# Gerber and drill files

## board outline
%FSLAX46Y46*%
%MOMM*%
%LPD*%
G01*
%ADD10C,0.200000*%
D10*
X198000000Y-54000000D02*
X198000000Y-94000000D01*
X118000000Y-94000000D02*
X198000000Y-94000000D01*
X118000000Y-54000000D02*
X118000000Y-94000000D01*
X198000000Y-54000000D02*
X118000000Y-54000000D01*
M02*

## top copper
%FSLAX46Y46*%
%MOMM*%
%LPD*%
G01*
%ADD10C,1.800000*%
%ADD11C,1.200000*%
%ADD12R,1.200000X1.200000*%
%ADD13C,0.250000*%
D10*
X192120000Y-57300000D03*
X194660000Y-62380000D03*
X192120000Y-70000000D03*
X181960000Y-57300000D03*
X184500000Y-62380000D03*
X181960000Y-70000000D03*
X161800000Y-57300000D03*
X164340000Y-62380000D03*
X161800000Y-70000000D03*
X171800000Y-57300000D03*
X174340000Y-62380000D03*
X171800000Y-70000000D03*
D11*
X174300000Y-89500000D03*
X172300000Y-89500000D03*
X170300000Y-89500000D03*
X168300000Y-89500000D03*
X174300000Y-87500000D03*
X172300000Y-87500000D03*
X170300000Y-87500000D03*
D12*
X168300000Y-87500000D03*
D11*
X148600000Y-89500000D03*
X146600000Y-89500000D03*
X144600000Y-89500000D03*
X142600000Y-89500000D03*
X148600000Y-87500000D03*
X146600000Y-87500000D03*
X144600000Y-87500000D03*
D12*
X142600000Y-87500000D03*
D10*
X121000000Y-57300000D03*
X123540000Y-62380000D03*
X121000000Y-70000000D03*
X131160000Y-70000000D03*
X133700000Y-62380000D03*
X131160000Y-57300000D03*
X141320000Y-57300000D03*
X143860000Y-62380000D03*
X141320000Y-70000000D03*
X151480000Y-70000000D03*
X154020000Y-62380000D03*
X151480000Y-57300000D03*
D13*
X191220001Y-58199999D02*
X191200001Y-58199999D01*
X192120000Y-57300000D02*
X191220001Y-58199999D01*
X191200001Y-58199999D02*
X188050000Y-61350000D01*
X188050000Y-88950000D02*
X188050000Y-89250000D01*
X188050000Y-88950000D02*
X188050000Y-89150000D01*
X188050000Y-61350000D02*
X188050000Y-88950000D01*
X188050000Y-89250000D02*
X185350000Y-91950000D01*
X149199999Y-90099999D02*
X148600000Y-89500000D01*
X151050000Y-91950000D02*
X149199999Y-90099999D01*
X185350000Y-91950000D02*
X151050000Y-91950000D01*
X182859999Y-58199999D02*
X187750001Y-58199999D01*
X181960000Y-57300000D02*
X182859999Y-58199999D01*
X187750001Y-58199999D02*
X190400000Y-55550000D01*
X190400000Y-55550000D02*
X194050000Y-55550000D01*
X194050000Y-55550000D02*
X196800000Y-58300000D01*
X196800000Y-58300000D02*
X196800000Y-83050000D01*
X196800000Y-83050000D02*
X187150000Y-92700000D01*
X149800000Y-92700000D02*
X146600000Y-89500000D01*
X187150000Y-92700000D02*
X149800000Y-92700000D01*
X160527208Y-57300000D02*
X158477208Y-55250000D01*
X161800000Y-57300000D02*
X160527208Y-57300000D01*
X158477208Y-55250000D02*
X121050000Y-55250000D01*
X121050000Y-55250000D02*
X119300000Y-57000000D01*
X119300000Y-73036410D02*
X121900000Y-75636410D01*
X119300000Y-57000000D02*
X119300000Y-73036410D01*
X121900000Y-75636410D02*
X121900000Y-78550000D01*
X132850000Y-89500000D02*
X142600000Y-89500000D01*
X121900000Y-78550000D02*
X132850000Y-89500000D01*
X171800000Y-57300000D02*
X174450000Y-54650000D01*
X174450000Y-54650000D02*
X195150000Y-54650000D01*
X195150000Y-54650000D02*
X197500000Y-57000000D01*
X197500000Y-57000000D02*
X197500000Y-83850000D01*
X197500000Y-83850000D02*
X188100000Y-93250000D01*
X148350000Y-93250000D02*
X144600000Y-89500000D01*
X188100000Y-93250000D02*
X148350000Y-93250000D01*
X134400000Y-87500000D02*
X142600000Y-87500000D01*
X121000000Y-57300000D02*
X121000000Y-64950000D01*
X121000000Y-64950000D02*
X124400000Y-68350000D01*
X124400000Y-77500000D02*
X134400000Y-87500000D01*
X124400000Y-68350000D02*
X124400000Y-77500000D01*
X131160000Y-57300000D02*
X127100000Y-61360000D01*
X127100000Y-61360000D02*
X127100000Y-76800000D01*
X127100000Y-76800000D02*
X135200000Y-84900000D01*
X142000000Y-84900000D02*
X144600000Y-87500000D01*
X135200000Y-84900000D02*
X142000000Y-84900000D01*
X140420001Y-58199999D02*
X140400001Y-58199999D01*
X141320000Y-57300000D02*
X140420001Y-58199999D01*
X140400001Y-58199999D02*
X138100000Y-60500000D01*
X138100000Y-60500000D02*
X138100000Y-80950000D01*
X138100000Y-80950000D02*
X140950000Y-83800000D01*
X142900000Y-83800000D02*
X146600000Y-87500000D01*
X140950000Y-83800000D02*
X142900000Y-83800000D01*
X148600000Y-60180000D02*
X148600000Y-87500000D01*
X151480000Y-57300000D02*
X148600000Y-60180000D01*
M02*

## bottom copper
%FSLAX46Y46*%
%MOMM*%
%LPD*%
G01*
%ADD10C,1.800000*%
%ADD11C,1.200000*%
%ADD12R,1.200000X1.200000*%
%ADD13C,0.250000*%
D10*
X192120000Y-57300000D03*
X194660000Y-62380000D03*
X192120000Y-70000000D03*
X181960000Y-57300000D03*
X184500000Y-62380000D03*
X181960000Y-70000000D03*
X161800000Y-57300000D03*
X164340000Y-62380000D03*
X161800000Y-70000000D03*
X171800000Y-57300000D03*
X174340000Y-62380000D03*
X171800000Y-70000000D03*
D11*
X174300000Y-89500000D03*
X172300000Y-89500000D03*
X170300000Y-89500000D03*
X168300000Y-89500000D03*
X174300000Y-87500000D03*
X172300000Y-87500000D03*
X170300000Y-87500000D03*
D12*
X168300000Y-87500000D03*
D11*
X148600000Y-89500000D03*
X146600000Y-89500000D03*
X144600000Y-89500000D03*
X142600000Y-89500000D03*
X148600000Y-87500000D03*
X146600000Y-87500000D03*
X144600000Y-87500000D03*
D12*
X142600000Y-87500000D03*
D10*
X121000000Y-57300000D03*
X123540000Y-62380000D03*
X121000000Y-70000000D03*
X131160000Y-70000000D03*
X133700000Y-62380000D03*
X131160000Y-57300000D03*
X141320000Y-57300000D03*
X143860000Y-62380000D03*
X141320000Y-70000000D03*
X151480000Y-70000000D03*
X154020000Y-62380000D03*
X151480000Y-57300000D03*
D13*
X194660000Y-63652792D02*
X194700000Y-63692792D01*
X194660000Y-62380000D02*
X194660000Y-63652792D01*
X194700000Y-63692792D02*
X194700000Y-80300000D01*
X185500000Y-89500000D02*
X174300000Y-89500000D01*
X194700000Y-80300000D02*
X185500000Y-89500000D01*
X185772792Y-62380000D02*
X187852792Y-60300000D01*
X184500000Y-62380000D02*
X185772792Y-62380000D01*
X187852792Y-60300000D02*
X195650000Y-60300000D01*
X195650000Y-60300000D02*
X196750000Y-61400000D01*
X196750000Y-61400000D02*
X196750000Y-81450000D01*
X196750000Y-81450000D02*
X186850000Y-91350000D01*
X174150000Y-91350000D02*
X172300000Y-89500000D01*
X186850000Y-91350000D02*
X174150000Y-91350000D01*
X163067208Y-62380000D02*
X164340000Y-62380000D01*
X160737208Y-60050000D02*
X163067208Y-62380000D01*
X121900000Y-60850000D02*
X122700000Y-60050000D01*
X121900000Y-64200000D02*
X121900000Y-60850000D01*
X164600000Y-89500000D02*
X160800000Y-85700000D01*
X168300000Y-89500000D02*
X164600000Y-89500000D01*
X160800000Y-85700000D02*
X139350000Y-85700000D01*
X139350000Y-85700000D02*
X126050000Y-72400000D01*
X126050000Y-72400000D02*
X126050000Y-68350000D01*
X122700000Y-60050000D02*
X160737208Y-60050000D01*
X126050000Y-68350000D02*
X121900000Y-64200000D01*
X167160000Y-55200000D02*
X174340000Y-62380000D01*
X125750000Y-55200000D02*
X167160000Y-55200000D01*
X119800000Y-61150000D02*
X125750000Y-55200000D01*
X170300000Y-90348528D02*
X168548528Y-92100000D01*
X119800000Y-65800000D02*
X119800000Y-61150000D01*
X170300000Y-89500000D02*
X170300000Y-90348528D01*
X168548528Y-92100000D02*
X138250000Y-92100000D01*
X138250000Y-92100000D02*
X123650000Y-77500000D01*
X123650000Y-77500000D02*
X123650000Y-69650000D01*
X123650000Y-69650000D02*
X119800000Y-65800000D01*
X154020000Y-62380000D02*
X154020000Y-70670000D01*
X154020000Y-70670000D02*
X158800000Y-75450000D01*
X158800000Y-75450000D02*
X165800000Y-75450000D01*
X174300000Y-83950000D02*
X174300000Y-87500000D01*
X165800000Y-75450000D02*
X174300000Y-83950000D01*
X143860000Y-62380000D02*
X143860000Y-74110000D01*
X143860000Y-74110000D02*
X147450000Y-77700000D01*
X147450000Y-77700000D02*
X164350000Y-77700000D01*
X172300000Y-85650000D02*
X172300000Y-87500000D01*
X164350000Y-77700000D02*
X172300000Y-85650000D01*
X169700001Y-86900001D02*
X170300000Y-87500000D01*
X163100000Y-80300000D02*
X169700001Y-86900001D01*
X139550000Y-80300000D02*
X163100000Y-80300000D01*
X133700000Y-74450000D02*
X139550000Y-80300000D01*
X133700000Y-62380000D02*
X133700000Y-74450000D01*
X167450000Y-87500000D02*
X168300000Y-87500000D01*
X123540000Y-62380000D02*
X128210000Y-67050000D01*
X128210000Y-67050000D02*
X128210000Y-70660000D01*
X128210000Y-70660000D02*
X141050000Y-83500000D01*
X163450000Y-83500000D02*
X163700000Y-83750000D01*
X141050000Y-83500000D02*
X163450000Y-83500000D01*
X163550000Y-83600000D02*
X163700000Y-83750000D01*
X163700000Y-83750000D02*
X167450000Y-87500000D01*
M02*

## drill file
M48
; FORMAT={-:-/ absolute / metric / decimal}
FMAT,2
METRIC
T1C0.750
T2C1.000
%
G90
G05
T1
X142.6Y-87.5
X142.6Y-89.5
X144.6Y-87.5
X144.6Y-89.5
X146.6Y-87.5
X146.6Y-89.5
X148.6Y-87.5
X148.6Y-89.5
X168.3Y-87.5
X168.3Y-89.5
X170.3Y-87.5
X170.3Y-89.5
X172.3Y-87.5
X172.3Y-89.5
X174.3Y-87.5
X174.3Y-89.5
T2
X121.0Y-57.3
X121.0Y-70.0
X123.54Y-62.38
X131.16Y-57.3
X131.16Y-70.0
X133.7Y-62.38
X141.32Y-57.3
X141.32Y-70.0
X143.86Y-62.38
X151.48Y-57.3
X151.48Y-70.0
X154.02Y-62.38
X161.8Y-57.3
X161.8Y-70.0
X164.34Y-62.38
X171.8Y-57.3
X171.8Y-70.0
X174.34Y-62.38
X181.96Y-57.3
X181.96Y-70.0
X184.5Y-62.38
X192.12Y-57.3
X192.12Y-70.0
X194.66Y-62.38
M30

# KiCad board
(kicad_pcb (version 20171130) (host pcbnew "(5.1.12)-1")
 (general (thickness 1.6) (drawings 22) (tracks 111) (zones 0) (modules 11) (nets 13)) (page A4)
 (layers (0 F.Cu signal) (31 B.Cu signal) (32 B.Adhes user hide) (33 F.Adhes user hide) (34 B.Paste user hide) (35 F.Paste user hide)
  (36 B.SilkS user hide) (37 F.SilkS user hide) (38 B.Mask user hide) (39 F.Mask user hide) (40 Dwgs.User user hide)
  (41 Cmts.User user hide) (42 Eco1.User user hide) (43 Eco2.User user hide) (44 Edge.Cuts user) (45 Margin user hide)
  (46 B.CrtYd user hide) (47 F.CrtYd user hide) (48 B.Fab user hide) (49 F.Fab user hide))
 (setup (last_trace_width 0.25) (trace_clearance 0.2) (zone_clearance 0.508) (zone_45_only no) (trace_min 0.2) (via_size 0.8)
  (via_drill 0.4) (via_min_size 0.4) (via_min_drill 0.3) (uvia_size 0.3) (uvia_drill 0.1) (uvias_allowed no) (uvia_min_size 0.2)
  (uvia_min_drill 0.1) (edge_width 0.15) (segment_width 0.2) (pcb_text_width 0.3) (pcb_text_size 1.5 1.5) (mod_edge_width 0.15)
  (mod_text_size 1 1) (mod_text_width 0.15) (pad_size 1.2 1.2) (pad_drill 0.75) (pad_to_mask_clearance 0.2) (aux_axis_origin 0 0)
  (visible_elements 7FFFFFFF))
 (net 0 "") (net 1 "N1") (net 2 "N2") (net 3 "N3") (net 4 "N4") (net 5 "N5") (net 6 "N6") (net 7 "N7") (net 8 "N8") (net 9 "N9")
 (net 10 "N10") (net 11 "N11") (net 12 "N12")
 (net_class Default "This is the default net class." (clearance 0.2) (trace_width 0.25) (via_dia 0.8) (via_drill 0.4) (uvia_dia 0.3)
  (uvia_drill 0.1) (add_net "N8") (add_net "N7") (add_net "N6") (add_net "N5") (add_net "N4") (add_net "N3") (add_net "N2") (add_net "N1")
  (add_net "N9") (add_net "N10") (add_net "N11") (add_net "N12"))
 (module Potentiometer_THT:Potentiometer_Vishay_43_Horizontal (layer F.Cu) (at 192.12 70 270)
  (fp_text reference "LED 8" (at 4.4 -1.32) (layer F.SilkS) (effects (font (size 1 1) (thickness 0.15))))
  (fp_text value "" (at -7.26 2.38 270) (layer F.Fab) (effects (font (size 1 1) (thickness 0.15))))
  (pad 3 thru_hole circle (at -12.7 0 270) (size 1.8 1.8) (drill 1) (layers *.Cu *.Mask))
  (pad 2 thru_hole circle (at -7.62 -2.54 270) (size 1.8 1.8) (drill 1) (layers *.Cu *.Mask))
  (pad 1 thru_hole circle (at 0 0 270) (size 1.8 1.8) (drill 1) (layers *.Cu *.Mask)))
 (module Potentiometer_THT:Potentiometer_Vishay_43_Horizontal (layer F.Cu) (at 181.96 70 270)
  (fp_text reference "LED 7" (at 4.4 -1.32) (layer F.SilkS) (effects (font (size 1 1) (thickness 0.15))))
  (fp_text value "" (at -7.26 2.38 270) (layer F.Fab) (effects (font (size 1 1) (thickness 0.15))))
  (pad 3 thru_hole circle (at -12.7 0 270) (size 1.8 1.8) (drill 1) (layers *.Cu *.Mask))
  (pad 2 thru_hole circle (at -7.62 -2.54 270) (size 1.8 1.8) (drill 1) (layers *.Cu *.Mask))
  (pad 1 thru_hole circle (at 0 0 270) (size 1.8 1.8) (drill 1) (layers *.Cu *.Mask)))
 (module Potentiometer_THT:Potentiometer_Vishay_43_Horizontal (layer F.Cu) (at 161.8 70 270)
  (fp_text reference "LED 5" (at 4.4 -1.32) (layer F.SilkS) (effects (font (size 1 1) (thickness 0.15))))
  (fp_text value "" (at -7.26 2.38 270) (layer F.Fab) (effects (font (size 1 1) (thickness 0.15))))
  (pad 3 thru_hole circle (at -12.7 0 270) (size 1.8 1.8) (drill 1) (layers *.Cu *.Mask))
  (pad 2 thru_hole circle (at -7.62 -2.54 270) (size 1.8 1.8) (drill 1) (layers *.Cu *.Mask))
  (pad 1 thru_hole circle (at 0 0 270) (size 1.8 1.8) (drill 1) (layers *.Cu *.Mask)))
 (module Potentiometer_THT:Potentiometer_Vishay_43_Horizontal (layer F.Cu) (at 171.8 70 270)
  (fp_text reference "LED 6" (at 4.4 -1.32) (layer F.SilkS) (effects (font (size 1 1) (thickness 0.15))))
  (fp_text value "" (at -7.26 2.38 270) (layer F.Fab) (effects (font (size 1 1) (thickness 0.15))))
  (pad 3 thru_hole circle (at -12.7 0 270) (size 1.8 1.8) (drill 1) (layers *.Cu *.Mask))
  (pad 2 thru_hole circle (at -7.62 -2.54 270) (size 1.8 1.8) (drill 1) (layers *.Cu *.Mask))
  (pad 1 thru_hole circle (at 0 0 270) (size 1.8 1.8) (drill 1) (layers *.Cu *.Mask)))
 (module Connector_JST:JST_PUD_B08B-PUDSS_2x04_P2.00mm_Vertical (layer F.Cu) (at 168.3 87.5)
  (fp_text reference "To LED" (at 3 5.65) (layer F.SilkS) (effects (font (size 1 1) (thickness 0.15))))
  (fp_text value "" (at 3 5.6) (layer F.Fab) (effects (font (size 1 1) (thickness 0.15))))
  (pad 8 thru_hole circle (at 6 2) (size 1.2 1.2) (drill 0.75) (layers *.Cu *.Mask))
  (pad 6 thru_hole circle (at 4 2) (size 1.2 1.2) (drill 0.75) (layers *.Cu *.Mask))
  (pad 4 thru_hole circle (at 2 2) (size 1.2 1.2) (drill 0.75) (layers *.Cu *.Mask))
  (pad 2 thru_hole circle (at 0 2) (size 1.2 1.2) (drill 0.75) (layers *.Cu *.Mask))
  (pad 7 thru_hole circle (at 6 0) (size 1.2 1.2) (drill 0.75) (layers *.Cu *.Mask) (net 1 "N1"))
  (pad 5 thru_hole circle (at 4 0) (size 1.2 1.2) (drill 0.75) (layers *.Cu *.Mask) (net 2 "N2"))
  (pad 3 thru_hole circle (at 2 0) (size 1.2 1.2) (drill 0.75) (layers *.Cu *.Mask) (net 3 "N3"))
  (pad 1 thru_hole rect (at 0 0) (size 1.2 1.2) (drill 0.75) (layers *.Cu *.Mask) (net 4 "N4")))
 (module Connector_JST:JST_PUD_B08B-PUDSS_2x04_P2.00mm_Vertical (layer F.Cu) (at 142.6 87.5)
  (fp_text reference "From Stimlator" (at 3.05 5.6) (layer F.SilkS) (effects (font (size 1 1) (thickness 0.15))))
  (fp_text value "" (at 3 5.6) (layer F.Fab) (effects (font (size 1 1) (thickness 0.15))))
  (pad 8 thru_hole circle (at 6 2) (size 1.2 1.2) (drill 0.75) (layers *.Cu *.Mask))
  (pad 6 thru_hole circle (at 4 2) (size 1.2 1.2) (drill 0.75) (layers *.Cu *.Mask))
  (pad 4 thru_hole circle (at 2 2) (size 1.2 1.2) (drill 0.75) (layers *.Cu *.Mask))
  (pad 2 thru_hole circle (at 0 2) (size 1.2 1.2) (drill 0.75) (layers *.Cu *.Mask))
  (pad 7 thru_hole circle (at 6 0) (size 1.2 1.2) (drill 0.75) (layers *.Cu *.Mask) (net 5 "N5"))
  (pad 5 thru_hole circle (at 4 0) (size 1.2 1.2) (drill 0.75) (layers *.Cu *.Mask) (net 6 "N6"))
  (pad 3 thru_hole circle (at 2 0) (size 1.2 1.2) (drill 0.75) (layers *.Cu *.Mask) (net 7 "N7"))
  (pad 1 thru_hole rect (at 0 0) (size 1.2 1.2) (drill 0.75) (layers *.Cu *.Mask) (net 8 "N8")))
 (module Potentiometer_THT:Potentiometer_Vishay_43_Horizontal (layer F.Cu) (at 121 70 270)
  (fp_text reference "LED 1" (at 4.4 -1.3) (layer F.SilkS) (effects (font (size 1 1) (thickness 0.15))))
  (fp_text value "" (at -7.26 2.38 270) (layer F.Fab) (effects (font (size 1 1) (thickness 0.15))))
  (pad 3 thru_hole circle (at -12.7 0 270) (size 1.8 1.8) (drill 1) (layers *.Cu *.Mask) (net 8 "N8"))
  (pad 2 thru_hole circle (at -7.62 -2.54 270) (size 1.8 1.8) (drill 1) (layers *.Cu *.Mask) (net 4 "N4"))
  (pad 1 thru_hole circle (at 0 0 270) (size 1.8 1.8) (drill 1) (layers *.Cu *.Mask) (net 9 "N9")))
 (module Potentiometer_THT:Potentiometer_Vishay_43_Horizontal (layer F.Cu) (at 131.16 70 270)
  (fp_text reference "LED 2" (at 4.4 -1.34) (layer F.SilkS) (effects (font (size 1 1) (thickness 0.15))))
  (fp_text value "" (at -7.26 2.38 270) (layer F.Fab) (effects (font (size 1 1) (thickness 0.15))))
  (pad 1 thru_hole circle (at 0 0 270) (size 1.8 1.8) (drill 1) (layers *.Cu *.Mask) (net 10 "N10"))
  (pad 2 thru_hole circle (at -7.62 -2.54 270) (size 1.8 1.8) (drill 1) (layers *.Cu *.Mask) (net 3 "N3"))
  (pad 3 thru_hole circle (at -12.7 0 270) (size 1.8 1.8) (drill 1) (layers *.Cu *.Mask) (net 7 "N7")))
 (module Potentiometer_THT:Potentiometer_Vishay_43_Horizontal (layer F.Cu) (at 141.32 70 270)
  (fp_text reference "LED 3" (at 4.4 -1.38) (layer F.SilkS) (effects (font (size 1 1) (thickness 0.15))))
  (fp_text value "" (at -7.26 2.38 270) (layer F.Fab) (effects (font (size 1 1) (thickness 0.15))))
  (pad 3 thru_hole circle (at -12.7 0 270) (size 1.8 1.8) (drill 1) (layers *.Cu *.Mask) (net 6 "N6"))
  (pad 2 thru_hole circle (at -7.62 -2.54 270) (size 1.8 1.8) (drill 1) (layers *.Cu *.Mask) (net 2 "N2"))
  (pad 1 thru_hole circle (at 0 0 270) (size 1.8 1.8) (drill 1) (layers *.Cu *.Mask) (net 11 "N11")))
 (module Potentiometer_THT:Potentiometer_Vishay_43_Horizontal (layer F.Cu) (at 151.48 70 270)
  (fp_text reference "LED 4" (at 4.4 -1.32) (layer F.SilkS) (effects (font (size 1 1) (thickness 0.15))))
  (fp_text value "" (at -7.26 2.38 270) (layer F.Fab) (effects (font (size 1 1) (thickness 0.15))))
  (pad 1 thru_hole circle (at 0 0 270) (size 1.8 1.8) (drill 1) (layers *.Cu *.Mask) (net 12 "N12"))
  (pad 2 thru_hole circle (at -7.62 -2.54 270) (size 1.8 1.8) (drill 1) (layers *.Cu *.Mask) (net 1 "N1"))
  (pad 3 thru_hole circle (at -12.7 0 270) (size 1.8 1.8) (drill 1) (layers *.Cu *.Mask) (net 5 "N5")))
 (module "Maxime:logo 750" (layer B.Cu) (at 157.7 76.7 180)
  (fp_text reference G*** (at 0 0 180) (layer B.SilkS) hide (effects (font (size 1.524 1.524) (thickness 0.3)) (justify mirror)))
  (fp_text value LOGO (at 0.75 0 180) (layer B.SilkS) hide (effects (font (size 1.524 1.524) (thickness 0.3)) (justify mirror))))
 (gr_line (start 198 54) (end 198 94) (layer Edge.Cuts) (width 0.2))
 (gr_line (start 118 94) (end 198 94) (layer Edge.Cuts) (width 0.2))
 (gr_line (start 118 54) (end 118 94) (layer Edge.Cuts) (width 0.2))
 (gr_line (start 198 54) (end 118 54) (layer Edge.Cuts) (width 0.2))
 (segment (start 191.220001 58.199999) (end 191.200001 58.199999) (width 0.25) (layer F.Cu) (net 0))
 (segment (start 192.12 57.3) (end 191.220001 58.199999) (width 0.25) (layer F.Cu) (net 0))
 (segment (start 191.200001 58.199999) (end 188.05 61.35) (width 0.25) (layer F.Cu) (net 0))
 (segment (start 188.05 88.95) (end 188.05 89.25) (width 0.25) (layer F.Cu) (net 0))
 (segment (start 188.05 88.95) (end 188.05 89.15) (width 0.25) (layer F.Cu) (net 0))
 (segment (start 188.05 61.35) (end 188.05 88.95) (width 0.25) (layer F.Cu) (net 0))
 (segment (start 188.05 89.25) (end 185.35 91.95) (width 0.25) (layer F.Cu) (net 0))
 (segment (start 149.199999 90.099999) (end 148.6 89.5) (width 0.25) (layer F.Cu) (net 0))
 (segment (start 151.05 91.95) (end 149.199999 90.099999) (width 0.25) (layer F.Cu) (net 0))
 (segment (start 185.35 91.95) (end 151.05 91.95) (width 0.25) (layer F.Cu) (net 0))
 (segment (start 182.859999 58.199999) (end 187.750001 58.199999) (width 0.25) (layer F.Cu) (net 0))
 (segment (start 181.96 57.3) (end 182.859999 58.199999) (width 0.25) (layer F.Cu) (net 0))
 (segment (start 187.750001 58.199999) (end 190.4 55.55) (width 0.25) (layer F.Cu) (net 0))
 (segment (start 190.4 55.55) (end 194.05 55.55) (width 0.25) (layer F.Cu) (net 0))
 (segment (start 194.05 55.55) (end 196.8 58.3) (width 0.25) (layer F.Cu) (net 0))
 (segment (start 196.8 58.3) (end 196.8 83.05) (width 0.25) (layer F.Cu) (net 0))
 (segment (start 196.8 83.05) (end 187.15 92.7) (width 0.25) (layer F.Cu) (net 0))
 (segment (start 149.8 92.7) (end 146.6 89.5) (width 0.25) (layer F.Cu) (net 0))
 (segment (start 187.15 92.7) (end 149.8 92.7) (width 0.25) (layer F.Cu) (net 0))
 (segment (start 160.527208 57.3) (end 158.477208 55.25) (width 0.25) (layer F.Cu) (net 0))
 (segment (start 161.8 57.3) (end 160.527208 57.3) (width 0.25) (layer F.Cu) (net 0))
 (segment (start 158.477208 55.25) (end 121.05 55.25) (width 0.25) (layer F.Cu) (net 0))
 (segment (start 121.05 55.25) (end 119.3 57) (width 0.25) (layer F.Cu) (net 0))
 (segment (start 119.3 73.03641) (end 121.9 75.63641) (width 0.25) (layer F.Cu) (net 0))
 (segment (start 119.3 57) (end 119.3 73.03641) (width 0.25) (layer F.Cu) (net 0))
 (segment (start 121.9 75.63641) (end 121.9 78.55) (width 0.25) (layer F.Cu) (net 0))
 (segment (start 132.85 89.5) (end 142.6 89.5) (width 0.25) (layer F.Cu) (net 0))
 (segment (start 121.9 78.55) (end 132.85 89.5) (width 0.25) (layer F.Cu) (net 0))
 (segment (start 171.8 57.3) (end 174.45 54.65) (width 0.25) (layer F.Cu) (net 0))
 (segment (start 174.45 54.65) (end 195.15 54.65) (width 0.25) (layer F.Cu) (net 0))
 (segment (start 195.15 54.65) (end 197.5 57) (width 0.25) (layer F.Cu) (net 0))
 (segment (start 197.5 57) (end 197.5 83.85) (width 0.25) (layer F.Cu) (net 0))
 (segment (start 197.5 83.85) (end 188.1 93.25) (width 0.25) (layer F.Cu) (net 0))
 (segment (start 148.35 93.25) (end 144.6 89.5) (width 0.25) (layer F.Cu) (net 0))
 (segment (start 188.1 93.25) (end 148.35 93.25) (width 0.25) (layer F.Cu) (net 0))
 (segment (start 194.66 63.652792) (end 194.7 63.692792) (width 0.25) (layer B.Cu) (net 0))
 (segment (start 194.66 62.38) (end 194.66 63.652792) (width 0.25) (layer B.Cu) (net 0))
 (segment (start 194.7 63.692792) (end 194.7 80.3) (width 0.25) (layer B.Cu) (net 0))
 (segment (start 185.5 89.5) (end 174.3 89.5) (width 0.25) (layer B.Cu) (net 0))
 (segment (start 194.7 80.3) (end 185.5 89.5) (width 0.25) (layer B.Cu) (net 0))
 (segment (start 185.772792 62.38) (end 187.852792 60.3) (width 0.25) (layer B.Cu) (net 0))
 (segment (start 184.5 62.38) (end 185.772792 62.38) (width 0.25) (layer B.Cu) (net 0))
 (segment (start 187.852792 60.3) (end 195.65 60.3) (width 0.25) (layer B.Cu) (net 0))
 (segment (start 195.65 60.3) (end 196.75 61.4) (width 0.25) (layer B.Cu) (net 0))
 (segment (start 196.75 61.4) (end 196.75 81.45) (width 0.25) (layer B.Cu) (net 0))
 (segment (start 196.75 81.45) (end 186.85 91.35) (width 0.25) (layer B.Cu) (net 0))
 (segment (start 174.15 91.35) (end 172.3 89.5) (width 0.25) (layer B.Cu) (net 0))
 (segment (start 186.85 91.35) (end 174.15 91.35) (width 0.25) (layer B.Cu) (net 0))
 (segment (start 163.067208 62.38) (end 164.34 62.38) (width 0.25) (layer B.Cu) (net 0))
 (segment (start 160.737208 60.05) (end 163.067208 62.38) (width 0.25) (layer B.Cu) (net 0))
 (segment (start 121.9 60.85) (end 122.7 60.05) (width 0.25) (layer B.Cu) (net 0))
 (segment (start 121.9 64.2) (end 121.9 60.85) (width 0.25) (layer B.Cu) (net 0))
 (segment (start 164.6 89.5) (end 160.8 85.7) (width 0.25) (layer B.Cu) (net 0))
 (segment (start 168.3 89.5) (end 164.6 89.5) (width 0.25) (layer B.Cu) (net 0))
 (segment (start 160.8 85.7) (end 139.35 85.7) (width 0.25) (layer B.Cu) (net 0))
 (segment (start 139.35 85.7) (end 126.05 72.4) (width 0.25) (layer B.Cu) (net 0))
 (segment (start 126.05 72.4) (end 126.05 68.35) (width 0.25) (layer B.Cu) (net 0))
 (segment (start 122.7 60.05) (end 160.737208 60.05) (width 0.25) (layer B.Cu) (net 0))
 (segment (start 126.05 68.35) (end 121.9 64.2) (width 0.25) (layer B.Cu) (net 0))
 (segment (start 167.16 55.2) (end 174.34 62.38) (width 0.25) (layer B.Cu) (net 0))
 (segment (start 125.75 55.2) (end 167.16 55.2) (width 0.25) (layer B.Cu) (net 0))
 (segment (start 119.8 61.15) (end 125.75 55.2) (width 0.25) (layer B.Cu) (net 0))
 (segment (start 170.3 90.348528) (end 168.548528 92.1) (width 0.25) (layer B.Cu) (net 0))
 (segment (start 119.8 65.8) (end 119.8 61.15) (width 0.25) (layer B.Cu) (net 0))
 (segment (start 170.3 89.5) (end 170.3 90.348528) (width 0.25) (layer B.Cu) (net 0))
 (segment (start 168.548528 92.1) (end 138.25 92.1) (width 0.25) (layer B.Cu) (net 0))
 (segment (start 138.25 92.1) (end 123.65 77.5) (width 0.25) (layer B.Cu) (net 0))
 (segment (start 123.65 77.5) (end 123.65 69.65) (width 0.25) (layer B.Cu) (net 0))
 (segment (start 123.65 69.65) (end 119.8 65.8) (width 0.25) (layer B.Cu) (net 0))
 (segment (start 134.4 87.5) (end 142.6 87.5) (width 0.25) (layer F.Cu) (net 8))
 (segment (start 121 57.3) (end 121 64.95) (width 0.25) (layer F.Cu) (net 8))
 (segment (start 121 64.95) (end 124.4 68.35) (width 0.25) (layer F.Cu) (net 8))
 (segment (start 124.4 77.5) (end 134.4 87.5) (width 0.25) (layer F.Cu) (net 8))
 (segment (start 124.4 68.35) (end 124.4 77.5) (width 0.25) (layer F.Cu) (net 8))
 (segment (start 131.16 57.3) (end 127.1 61.36) (width 0.25) (layer F.Cu) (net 7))
 (segment (start 127.1 61.36) (end 127.1 76.8) (width 0.25) (layer F.Cu) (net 7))
 (segment (start 127.1 76.8) (end 135.2 84.9) (width 0.25) (layer F.Cu) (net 7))
 (segment (start 142 84.9) (end 144.6 87.5) (width 0.25) (layer F.Cu) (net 7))
 (segment (start 135.2 84.9) (end 142 84.9) (width 0.25) (layer F.Cu) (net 7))
 (segment (start 140.420001 58.199999) (end 140.400001 58.199999) (width 0.25) (layer F.Cu) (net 6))
 (segment (start 141.32 57.3) (end 140.420001 58.199999) (width 0.25) (layer F.Cu) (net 6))
 (segment (start 140.400001 58.199999) (end 138.1 60.5) (width 0.25) (layer F.Cu) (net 6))
 (segment (start 138.1 60.5) (end 138.1 80.95) (width 0.25) (layer F.Cu) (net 6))
 (segment (start 138.1 80.95) (end 140.95 83.8) (width 0.25) (layer F.Cu) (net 6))
 (segment (start 142.9 83.8) (end 146.6 87.5) (width 0.25) (layer F.Cu) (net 6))
 (segment (start 140.95 83.8) (end 142.9 83.8) (width 0.25) (layer F.Cu) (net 6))
 (segment (start 148.6 60.18) (end 148.6 87.5) (width 0.25) (layer F.Cu) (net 5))
 (segment (start 151.48 57.3) (end 148.6 60.18) (width 0.25) (layer F.Cu) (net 5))
 (segment (start 154.02 62.38) (end 154.02 70.67) (width 0.25) (layer B.Cu) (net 1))
 (segment (start 154.02 70.67) (end 158.8 75.45) (width 0.25) (layer B.Cu) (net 1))
 (segment (start 158.8 75.45) (end 165.8 75.45) (width 0.25) (layer B.Cu) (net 1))
 (segment (start 174.3 83.95) (end 174.3 87.5) (width 0.25) (layer B.Cu) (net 1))
 (segment (start 165.8 75.45) (end 174.3 83.95) (width 0.25) (layer B.Cu) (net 1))
 (segment (start 143.86 62.38) (end 143.86 74.11) (width 0.25) (layer B.Cu) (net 2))
 (segment (start 143.86 74.11) (end 147.45 77.7) (width 0.25) (layer B.Cu) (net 2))
 (segment (start 147.45 77.7) (end 164.35 77.7) (width 0.25) (layer B.Cu) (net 2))
 (segment (start 172.3 85.65) (end 172.3 87.5) (width 0.25) (layer B.Cu) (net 2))
 (segment (start 164.35 77.7) (end 172.3 85.65) (width 0.25) (layer B.Cu) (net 2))
 (segment (start 169.700001 86.900001) (end 170.3 87.5) (width 0.25) (layer B.Cu) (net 3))
 (segment (start 163.1 80.3) (end 169.700001 86.900001) (width 0.25) (layer B.Cu) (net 3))
 (segment (start 139.55 80.3) (end 163.1 80.3) (width 0.25) (layer B.Cu) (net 3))
 (segment (start 133.7 74.45) (end 139.55 80.3) (width 0.25) (layer B.Cu) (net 3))
 (segment (start 133.7 62.38) (end 133.7 74.45) (width 0.25) (layer B.Cu) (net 3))
 (segment (start 167.45 87.5) (end 168.3 87.5) (width 0.25) (layer B.Cu) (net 4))
 (segment (start 123.54 62.38) (end 128.21 67.05) (width 0.25) (layer B.Cu) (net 4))
 (segment (start 128.21 67.05) (end 128.21 70.66) (width 0.25) (layer B.Cu) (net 4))
 (segment (start 128.21 70.66) (end 141.05 83.5) (width 0.25) (layer B.Cu) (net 4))
 (segment (start 163.45 83.5) (end 163.7 83.75) (width 0.25) (layer B.Cu) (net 4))
 (segment (start 141.05 83.5) (end 163.45 83.5) (width 0.25) (layer B.Cu) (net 4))
 (segment (start 163.55 83.6) (end 163.7 83.75) (width 0.25) (layer B.Cu) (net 4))
 (segment (start 163.7 83.75) (end 167.45 87.5) (width 0.25) (layer B.Cu) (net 4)))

